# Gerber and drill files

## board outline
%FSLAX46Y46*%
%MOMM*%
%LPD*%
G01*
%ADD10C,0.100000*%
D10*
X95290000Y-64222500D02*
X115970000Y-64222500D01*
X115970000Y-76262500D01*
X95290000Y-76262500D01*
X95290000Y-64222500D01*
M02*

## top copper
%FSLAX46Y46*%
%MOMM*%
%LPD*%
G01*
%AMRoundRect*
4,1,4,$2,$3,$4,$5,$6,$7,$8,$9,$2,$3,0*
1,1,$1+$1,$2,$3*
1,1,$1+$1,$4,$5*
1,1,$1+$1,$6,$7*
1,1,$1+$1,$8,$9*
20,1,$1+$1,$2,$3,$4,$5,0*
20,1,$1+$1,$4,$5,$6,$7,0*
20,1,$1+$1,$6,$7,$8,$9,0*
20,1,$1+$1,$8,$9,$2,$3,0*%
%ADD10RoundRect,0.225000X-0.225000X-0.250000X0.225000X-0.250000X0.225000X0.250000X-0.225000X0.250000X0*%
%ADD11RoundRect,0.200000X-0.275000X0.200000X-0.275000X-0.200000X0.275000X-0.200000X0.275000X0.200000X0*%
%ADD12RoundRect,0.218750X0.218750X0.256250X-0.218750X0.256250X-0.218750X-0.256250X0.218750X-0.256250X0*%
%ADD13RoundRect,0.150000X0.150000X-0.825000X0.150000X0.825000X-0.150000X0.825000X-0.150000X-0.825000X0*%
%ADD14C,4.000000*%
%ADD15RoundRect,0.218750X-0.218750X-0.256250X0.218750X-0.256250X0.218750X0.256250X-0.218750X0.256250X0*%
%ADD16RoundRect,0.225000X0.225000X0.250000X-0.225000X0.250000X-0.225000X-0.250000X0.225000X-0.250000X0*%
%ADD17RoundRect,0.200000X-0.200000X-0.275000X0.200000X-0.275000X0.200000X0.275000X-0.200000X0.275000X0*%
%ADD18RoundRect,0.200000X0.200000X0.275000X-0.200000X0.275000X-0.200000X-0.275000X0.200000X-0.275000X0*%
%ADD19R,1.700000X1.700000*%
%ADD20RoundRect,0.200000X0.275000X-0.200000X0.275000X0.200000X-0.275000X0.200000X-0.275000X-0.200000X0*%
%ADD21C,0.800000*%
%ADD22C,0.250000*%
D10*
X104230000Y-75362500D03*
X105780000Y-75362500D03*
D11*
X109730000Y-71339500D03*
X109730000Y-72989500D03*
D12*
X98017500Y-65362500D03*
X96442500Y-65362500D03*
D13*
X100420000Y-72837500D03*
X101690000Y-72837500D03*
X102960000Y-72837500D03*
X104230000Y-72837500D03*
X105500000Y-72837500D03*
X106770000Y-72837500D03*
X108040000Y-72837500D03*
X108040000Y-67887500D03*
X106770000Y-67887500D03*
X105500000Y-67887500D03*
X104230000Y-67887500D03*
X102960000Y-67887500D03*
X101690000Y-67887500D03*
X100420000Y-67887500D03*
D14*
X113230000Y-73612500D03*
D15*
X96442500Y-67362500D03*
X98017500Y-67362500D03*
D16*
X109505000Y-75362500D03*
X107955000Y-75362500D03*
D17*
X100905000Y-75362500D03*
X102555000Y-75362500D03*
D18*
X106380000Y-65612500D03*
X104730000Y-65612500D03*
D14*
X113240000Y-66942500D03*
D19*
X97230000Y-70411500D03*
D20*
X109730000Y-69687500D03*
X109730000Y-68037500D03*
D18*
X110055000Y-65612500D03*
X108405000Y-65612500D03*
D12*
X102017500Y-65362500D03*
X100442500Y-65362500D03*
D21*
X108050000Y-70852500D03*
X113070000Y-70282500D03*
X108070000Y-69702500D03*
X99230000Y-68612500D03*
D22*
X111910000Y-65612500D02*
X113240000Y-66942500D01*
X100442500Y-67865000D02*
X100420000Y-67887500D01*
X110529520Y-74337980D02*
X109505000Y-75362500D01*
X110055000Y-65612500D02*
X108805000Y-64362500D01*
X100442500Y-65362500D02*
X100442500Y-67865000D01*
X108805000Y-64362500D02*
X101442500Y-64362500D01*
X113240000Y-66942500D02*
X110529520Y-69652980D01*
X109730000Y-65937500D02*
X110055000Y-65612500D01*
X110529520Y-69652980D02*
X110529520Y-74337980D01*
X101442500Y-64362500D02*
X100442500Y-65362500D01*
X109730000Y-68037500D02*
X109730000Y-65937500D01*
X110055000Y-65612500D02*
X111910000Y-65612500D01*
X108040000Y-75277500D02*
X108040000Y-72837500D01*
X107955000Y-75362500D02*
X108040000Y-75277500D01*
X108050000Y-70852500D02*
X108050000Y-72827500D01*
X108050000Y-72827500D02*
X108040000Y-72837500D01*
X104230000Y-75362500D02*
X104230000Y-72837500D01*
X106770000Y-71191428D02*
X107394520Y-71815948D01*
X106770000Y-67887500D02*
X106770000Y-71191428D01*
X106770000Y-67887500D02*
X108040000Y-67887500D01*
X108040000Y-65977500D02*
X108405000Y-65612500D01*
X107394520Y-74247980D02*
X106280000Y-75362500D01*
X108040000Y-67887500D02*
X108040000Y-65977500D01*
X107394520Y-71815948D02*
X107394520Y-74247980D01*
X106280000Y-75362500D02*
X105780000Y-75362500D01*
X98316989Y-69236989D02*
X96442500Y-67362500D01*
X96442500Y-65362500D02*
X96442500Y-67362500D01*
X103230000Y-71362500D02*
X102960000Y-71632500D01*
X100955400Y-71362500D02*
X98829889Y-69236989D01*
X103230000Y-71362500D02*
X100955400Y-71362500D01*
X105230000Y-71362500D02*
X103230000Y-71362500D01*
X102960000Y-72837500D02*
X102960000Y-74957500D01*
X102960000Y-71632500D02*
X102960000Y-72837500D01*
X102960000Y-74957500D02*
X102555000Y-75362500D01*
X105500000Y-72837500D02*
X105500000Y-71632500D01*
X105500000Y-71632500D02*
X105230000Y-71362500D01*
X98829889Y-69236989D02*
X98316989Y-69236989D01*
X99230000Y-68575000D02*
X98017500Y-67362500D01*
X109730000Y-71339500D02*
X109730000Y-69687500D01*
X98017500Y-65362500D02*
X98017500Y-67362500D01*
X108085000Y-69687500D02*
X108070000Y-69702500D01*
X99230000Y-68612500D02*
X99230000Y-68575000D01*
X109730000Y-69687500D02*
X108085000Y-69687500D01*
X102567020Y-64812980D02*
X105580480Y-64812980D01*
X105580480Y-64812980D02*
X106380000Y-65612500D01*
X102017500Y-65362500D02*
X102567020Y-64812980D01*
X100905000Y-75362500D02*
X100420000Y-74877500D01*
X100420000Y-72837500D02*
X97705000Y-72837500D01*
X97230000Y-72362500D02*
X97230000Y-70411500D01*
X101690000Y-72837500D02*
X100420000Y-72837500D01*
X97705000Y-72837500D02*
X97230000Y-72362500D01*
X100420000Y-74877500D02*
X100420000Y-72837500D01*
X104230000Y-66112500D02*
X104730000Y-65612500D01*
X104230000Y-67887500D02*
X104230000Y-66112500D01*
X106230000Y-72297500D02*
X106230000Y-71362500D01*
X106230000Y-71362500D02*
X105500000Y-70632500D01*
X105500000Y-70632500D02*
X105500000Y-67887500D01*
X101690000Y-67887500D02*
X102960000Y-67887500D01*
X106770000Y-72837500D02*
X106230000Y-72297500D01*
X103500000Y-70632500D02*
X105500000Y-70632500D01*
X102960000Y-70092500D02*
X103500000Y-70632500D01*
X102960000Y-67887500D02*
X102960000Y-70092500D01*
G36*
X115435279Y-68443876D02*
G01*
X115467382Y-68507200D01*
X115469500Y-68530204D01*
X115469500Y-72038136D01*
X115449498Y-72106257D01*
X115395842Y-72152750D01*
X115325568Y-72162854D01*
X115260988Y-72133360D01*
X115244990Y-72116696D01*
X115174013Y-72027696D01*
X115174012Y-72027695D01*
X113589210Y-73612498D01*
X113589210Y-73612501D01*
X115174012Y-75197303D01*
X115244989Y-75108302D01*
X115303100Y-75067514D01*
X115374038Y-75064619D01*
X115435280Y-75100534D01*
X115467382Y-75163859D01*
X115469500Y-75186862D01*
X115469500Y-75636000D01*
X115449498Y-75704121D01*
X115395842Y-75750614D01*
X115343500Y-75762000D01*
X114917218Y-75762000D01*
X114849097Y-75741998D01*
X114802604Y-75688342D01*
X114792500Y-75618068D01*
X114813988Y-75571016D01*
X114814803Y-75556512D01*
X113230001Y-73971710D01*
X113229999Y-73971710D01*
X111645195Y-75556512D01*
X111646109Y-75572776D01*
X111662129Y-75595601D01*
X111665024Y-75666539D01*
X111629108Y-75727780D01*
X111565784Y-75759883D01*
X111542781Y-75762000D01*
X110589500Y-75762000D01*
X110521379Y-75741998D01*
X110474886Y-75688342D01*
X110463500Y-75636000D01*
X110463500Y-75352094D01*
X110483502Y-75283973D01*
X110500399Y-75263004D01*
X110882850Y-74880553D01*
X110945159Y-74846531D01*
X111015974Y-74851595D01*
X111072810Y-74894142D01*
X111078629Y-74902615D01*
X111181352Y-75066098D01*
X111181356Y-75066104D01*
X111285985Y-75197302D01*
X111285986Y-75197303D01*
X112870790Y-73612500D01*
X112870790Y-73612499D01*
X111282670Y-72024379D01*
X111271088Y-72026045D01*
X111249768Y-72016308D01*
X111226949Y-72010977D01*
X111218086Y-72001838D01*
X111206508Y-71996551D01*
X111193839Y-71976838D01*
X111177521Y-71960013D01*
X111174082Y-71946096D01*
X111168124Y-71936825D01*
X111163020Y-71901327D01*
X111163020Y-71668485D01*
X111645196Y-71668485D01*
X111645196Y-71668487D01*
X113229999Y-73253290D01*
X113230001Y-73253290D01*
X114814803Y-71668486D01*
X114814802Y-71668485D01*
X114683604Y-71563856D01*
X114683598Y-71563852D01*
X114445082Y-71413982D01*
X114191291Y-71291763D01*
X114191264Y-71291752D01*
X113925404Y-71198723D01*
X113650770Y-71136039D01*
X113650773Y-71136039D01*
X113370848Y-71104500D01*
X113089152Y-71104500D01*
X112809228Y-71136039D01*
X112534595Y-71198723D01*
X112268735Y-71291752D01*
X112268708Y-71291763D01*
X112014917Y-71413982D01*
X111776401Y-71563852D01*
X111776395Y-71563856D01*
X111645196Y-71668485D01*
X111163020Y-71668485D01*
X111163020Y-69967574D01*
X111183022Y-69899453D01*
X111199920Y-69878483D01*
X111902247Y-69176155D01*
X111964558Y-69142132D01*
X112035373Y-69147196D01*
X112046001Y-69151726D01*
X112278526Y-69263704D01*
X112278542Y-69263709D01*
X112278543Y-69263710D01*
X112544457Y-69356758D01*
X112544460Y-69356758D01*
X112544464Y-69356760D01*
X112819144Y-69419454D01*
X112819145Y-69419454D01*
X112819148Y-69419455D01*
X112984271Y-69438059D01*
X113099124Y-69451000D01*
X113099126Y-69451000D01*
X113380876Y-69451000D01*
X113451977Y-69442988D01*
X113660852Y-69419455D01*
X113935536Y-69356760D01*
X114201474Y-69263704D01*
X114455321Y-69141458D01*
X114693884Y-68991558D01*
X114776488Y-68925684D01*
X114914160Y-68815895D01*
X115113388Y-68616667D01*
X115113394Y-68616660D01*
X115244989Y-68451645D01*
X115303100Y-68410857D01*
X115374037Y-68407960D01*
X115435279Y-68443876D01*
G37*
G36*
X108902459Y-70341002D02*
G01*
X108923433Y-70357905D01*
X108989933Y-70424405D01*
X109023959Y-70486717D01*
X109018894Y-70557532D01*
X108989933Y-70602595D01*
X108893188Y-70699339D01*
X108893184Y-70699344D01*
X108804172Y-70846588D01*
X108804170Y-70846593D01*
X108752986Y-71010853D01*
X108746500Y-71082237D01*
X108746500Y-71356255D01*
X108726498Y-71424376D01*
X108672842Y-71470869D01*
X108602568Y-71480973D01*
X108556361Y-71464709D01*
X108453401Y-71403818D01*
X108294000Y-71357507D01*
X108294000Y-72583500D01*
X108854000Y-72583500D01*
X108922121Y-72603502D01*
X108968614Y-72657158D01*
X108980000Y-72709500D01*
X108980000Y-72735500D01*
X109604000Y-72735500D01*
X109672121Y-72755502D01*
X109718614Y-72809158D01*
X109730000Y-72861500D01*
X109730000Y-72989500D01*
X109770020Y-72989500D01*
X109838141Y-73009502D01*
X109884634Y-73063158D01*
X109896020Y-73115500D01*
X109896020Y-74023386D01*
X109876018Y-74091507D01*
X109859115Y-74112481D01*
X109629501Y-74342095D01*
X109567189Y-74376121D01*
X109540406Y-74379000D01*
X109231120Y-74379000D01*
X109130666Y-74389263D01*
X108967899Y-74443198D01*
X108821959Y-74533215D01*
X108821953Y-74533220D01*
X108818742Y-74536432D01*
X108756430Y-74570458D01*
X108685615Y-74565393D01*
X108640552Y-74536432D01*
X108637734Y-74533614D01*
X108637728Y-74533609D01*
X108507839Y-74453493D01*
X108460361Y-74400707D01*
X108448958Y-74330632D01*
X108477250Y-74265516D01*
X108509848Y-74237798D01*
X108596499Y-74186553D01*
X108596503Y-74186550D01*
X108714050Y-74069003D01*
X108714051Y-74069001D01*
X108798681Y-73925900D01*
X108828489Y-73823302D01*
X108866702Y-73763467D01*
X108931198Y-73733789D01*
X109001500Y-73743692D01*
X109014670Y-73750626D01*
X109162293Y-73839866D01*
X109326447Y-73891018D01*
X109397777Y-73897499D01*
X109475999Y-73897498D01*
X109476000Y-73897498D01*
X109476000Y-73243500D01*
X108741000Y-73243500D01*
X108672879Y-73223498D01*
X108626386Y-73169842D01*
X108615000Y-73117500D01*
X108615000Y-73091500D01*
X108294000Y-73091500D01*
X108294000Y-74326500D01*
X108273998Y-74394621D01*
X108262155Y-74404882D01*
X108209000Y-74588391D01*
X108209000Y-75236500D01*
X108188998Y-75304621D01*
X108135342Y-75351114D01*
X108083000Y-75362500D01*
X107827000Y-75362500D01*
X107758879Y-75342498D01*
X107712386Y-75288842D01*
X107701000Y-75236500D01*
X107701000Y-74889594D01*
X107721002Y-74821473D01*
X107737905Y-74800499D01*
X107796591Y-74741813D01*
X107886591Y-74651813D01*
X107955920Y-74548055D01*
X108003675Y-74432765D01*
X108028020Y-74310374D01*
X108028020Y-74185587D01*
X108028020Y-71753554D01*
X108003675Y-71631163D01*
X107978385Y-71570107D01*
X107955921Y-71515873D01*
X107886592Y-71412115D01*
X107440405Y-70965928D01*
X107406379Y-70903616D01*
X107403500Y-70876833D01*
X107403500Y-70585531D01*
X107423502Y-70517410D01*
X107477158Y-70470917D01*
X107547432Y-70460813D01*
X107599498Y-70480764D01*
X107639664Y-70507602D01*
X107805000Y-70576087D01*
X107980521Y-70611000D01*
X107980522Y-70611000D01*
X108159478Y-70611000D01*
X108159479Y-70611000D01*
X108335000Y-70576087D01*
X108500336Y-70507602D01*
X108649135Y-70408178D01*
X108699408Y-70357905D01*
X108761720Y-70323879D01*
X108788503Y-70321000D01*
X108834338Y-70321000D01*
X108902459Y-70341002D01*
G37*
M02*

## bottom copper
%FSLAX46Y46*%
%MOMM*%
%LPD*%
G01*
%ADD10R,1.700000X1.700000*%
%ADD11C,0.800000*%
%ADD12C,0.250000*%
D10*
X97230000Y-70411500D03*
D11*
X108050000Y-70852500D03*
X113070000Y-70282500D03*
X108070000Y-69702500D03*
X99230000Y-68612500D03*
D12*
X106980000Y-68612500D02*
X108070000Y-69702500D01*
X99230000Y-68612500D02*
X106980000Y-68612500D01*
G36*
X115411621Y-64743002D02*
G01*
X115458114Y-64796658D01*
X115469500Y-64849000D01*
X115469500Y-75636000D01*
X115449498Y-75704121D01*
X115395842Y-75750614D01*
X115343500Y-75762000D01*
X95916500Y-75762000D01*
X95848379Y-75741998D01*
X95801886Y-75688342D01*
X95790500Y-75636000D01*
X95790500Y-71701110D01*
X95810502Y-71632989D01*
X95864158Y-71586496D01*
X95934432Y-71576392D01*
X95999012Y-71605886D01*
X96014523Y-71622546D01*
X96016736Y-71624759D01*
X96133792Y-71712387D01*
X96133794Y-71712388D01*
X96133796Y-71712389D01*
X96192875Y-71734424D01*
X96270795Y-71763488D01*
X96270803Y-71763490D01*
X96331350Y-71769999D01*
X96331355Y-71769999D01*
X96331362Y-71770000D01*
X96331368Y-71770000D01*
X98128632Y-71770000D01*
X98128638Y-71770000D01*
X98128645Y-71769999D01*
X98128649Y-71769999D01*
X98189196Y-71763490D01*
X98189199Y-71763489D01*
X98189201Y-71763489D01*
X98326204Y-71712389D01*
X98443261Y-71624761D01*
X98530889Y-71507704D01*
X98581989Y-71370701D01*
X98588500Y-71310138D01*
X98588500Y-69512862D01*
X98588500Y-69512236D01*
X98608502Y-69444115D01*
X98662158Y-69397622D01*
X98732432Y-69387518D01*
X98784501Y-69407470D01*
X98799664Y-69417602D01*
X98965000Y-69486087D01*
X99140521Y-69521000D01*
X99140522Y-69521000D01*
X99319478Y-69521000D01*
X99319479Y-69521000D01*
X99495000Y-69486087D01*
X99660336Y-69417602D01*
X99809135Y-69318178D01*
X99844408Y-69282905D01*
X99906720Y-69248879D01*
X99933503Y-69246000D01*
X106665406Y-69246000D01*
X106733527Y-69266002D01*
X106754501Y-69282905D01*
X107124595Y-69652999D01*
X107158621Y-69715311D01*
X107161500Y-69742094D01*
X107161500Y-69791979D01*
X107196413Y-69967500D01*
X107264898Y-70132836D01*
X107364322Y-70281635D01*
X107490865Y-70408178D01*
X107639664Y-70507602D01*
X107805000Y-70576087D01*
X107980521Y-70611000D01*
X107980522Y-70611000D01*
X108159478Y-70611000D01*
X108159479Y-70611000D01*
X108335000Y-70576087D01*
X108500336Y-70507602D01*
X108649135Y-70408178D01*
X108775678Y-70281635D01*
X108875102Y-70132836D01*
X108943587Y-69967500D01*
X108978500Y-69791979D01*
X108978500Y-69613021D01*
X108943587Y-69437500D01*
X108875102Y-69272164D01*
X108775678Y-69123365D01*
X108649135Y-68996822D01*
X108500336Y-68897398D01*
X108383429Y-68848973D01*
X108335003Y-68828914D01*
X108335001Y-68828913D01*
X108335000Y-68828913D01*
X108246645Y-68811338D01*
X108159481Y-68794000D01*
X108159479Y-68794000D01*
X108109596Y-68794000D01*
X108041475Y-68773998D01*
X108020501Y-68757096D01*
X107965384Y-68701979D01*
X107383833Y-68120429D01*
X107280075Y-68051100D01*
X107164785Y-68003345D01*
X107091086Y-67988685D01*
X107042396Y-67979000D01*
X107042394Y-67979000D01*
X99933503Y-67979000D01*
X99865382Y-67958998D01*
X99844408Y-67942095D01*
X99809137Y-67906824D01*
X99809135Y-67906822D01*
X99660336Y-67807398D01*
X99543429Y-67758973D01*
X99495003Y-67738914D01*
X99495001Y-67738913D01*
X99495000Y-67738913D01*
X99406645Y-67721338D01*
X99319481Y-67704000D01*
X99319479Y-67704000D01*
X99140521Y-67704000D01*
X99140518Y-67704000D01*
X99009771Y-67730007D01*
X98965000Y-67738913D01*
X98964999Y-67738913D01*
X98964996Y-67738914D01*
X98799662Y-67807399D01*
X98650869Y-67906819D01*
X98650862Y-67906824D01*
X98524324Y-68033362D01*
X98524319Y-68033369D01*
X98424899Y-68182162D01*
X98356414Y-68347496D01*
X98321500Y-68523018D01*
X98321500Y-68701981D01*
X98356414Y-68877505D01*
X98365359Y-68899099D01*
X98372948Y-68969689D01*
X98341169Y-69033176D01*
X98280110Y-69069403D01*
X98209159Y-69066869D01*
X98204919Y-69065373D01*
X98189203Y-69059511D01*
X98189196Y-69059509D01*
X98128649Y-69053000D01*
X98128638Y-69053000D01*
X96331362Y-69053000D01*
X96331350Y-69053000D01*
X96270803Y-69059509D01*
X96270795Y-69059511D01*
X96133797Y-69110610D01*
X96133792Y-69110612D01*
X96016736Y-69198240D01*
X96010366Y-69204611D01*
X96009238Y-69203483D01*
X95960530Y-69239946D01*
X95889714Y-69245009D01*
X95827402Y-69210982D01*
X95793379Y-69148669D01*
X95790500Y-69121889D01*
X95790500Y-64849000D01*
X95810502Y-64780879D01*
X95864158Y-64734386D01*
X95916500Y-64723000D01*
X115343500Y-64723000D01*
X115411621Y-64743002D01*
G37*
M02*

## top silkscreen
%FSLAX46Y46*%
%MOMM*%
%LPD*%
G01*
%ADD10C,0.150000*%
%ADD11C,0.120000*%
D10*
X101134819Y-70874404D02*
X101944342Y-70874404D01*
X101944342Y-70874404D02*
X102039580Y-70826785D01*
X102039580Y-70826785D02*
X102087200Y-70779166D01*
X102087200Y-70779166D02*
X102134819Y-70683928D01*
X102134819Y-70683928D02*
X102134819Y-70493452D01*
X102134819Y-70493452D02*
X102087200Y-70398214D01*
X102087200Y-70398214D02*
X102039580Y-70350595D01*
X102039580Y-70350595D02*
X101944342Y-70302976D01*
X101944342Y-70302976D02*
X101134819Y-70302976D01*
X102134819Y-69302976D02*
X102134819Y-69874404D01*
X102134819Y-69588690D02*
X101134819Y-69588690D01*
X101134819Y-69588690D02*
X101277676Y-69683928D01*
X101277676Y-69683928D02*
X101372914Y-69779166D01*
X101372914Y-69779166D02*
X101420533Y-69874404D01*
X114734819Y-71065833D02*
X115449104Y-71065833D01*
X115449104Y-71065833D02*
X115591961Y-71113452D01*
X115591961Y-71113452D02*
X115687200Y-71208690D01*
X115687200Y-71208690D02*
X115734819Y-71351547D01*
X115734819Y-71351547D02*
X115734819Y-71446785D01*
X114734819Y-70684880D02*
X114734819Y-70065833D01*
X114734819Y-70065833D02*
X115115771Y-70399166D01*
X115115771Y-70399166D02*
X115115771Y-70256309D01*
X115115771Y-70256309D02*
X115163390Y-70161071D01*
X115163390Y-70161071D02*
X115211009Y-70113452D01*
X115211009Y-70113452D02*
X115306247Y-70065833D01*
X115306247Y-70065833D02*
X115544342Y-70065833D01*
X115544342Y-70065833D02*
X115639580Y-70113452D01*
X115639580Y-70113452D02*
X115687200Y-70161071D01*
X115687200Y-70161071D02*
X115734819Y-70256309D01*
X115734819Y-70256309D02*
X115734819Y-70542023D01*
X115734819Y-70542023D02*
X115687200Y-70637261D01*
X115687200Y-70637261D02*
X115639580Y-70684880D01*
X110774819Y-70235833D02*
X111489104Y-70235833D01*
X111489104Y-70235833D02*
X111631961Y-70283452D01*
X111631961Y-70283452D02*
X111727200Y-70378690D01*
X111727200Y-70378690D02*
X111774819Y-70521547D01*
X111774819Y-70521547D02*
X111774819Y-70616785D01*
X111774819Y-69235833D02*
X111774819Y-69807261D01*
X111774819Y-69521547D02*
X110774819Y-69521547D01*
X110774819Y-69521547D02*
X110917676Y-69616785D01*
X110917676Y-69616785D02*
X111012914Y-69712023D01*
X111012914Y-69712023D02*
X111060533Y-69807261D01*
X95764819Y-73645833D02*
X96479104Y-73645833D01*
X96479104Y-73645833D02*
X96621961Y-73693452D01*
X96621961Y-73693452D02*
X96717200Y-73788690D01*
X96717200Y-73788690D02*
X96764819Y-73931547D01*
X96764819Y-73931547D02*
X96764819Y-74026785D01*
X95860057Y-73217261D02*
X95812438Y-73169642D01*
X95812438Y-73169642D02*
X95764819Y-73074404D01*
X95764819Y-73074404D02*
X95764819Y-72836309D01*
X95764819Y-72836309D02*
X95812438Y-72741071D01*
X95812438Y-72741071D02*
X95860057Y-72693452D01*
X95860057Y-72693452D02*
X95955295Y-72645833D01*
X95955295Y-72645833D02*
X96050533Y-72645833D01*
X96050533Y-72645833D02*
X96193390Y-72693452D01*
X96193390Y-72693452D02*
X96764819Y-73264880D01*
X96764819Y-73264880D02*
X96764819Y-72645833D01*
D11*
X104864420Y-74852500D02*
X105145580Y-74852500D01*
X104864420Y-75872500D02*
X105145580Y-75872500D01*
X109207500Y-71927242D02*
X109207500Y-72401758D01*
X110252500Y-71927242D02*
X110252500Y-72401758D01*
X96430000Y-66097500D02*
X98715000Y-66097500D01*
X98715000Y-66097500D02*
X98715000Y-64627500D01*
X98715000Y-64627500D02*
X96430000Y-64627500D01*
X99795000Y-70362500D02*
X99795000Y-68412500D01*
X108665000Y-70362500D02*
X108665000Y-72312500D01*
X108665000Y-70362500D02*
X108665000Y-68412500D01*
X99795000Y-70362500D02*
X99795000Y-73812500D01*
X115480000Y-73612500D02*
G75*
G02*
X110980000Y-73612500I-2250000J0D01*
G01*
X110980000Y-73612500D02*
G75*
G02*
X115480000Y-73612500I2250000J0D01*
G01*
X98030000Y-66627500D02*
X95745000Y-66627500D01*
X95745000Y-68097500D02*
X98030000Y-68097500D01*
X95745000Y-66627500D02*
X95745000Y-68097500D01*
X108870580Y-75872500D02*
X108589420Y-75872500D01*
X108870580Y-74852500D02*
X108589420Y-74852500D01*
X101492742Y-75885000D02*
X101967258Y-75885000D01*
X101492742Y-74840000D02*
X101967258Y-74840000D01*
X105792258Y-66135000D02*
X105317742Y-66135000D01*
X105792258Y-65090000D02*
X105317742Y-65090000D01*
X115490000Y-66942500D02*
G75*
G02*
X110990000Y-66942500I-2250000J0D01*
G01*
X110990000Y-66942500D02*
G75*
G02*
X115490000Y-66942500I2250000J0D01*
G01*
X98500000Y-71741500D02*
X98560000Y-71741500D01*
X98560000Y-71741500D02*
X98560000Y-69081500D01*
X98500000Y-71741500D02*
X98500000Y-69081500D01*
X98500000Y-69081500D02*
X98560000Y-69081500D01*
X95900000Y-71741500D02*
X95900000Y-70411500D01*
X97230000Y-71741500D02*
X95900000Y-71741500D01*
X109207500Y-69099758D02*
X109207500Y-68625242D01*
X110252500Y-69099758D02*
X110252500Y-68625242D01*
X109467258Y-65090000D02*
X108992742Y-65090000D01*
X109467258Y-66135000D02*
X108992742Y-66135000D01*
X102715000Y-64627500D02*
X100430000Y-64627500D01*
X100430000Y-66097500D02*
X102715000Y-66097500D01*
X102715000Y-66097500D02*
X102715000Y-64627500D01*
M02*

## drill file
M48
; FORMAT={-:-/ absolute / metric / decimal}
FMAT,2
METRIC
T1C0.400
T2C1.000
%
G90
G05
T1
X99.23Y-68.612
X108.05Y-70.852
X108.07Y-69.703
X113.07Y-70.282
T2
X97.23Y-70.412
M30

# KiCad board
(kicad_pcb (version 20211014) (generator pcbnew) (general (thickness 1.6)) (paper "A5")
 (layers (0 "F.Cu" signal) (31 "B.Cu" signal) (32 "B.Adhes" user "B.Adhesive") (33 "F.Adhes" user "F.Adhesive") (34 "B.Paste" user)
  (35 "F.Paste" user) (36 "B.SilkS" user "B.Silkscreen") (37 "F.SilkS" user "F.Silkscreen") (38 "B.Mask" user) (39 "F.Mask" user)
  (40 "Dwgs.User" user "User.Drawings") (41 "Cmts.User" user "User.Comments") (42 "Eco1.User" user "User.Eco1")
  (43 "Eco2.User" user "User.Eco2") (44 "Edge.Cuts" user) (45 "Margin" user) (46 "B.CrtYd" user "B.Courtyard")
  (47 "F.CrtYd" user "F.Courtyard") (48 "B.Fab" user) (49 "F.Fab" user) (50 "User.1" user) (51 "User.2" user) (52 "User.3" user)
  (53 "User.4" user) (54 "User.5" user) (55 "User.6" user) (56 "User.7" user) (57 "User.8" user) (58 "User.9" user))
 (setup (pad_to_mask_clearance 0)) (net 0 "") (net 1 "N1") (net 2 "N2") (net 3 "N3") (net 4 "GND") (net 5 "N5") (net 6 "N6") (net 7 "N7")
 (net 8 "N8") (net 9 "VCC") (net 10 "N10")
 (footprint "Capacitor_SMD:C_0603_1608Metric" (layer "F.Cu") (at 105.005 75.3625)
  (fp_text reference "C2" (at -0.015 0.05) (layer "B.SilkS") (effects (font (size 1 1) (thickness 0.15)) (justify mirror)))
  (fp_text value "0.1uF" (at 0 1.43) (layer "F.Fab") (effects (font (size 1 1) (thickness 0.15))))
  (fp_line (start -0.14058 -0.51) (end 0.14058 -0.51) (layer "F.SilkS") (width 0.12))
  (fp_line (start -0.14058 0.51) (end 0.14058 0.51) (layer "F.SilkS") (width 0.12))
  (pad "1" smd roundrect locked (at -0.775 0) (size 0.9 0.95) (layers "F.Cu" "F.Paste" "F.Mask") (roundrect_rratio 0.25) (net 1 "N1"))
  (pad "2" smd roundrect locked (at 0.775 0) (size 0.9 0.95) (layers "F.Cu" "F.Paste" "F.Mask") (roundrect_rratio 0.25) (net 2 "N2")))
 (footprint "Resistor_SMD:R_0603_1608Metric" (layer "F.Cu") (at 109.73 72.1645 -90)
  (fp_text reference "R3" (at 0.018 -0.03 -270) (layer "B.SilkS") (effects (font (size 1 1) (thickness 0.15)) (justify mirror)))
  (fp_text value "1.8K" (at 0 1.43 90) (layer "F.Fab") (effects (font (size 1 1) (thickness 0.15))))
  (fp_line (start -0.237258 0.5225) (end 0.237258 0.5225) (layer "F.SilkS") (width 0.12))
  (fp_line (start -0.237258 -0.5225) (end 0.237258 -0.5225) (layer "F.SilkS") (width 0.12))
  (pad "1" smd roundrect locked (at -0.825 0 270) (size 0.8 0.95) (layers "F.Cu" "F.Paste" "F.Mask") (roundrect_rratio 0.25) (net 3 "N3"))
  (pad "2" smd roundrect locked (at 0.825 0 270) (size 0.8 0.95) (layers "F.Cu" "F.Paste" "F.Mask") (roundrect_rratio 0.25) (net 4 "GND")))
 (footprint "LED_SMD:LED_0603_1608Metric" (layer "F.Cu") (at 97.23 65.3625 180)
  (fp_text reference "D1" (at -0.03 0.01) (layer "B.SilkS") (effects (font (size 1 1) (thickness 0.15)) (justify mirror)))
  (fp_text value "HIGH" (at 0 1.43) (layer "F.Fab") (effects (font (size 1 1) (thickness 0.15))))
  (fp_line (start 0.8 -0.735) (end -1.485 -0.735) (layer "F.SilkS") (width 0.12))
  (fp_line (start -1.485 -0.735) (end -1.485 0.735) (layer "F.SilkS") (width 0.12))
  (fp_line (start -1.485 0.735) (end 0.8 0.735) (layer "F.SilkS") (width 0.12))
  (pad "1" smd roundrect locked (at -0.7875 0 180) (size 0.875 0.95) (layers "F.Cu" "F.Paste" "F.Mask") (roundrect_rratio 0.25) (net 3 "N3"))
  (pad "2" smd roundrect locked (at 0.7875 0 180) (size 0.875 0.95) (layers "F.Cu" "F.Paste" "F.Mask") (roundrect_rratio 0.25) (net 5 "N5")))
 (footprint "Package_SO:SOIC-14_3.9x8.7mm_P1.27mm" (layer "F.Cu") (at 104.23 70.3625 90)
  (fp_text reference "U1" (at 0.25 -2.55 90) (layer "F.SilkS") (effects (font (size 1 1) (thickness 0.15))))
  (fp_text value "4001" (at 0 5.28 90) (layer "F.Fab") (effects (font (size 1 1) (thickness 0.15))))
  (fp_line (start 0 -4.435) (end 1.95 -4.435) (layer "F.SilkS") (width 0.12))
  (fp_line (start 0 4.435) (end -1.95 4.435) (layer "F.SilkS") (width 0.12))
  (fp_line (start 0 4.435) (end 1.95 4.435) (layer "F.SilkS") (width 0.12))
  (fp_line (start 0 -4.435) (end -3.45 -4.435) (layer "F.SilkS") (width 0.12))
  (pad "1" smd roundrect locked (at -2.475 -3.81 90) (size 1.95 0.6) (layers "F.Cu" "F.Paste" "F.Mask") (roundrect_rratio 0.25) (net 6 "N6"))
  (pad "2" smd roundrect locked (at -2.475 -2.54 90) (size 1.95 0.6) (layers "F.Cu" "F.Paste" "F.Mask") (roundrect_rratio 0.25) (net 6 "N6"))
  (pad "3" smd roundrect locked (at -2.475 -1.27 90) (size 1.95 0.6) (layers "F.Cu" "F.Paste" "F.Mask") (roundrect_rratio 0.25) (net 5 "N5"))
  (pad "4" smd roundrect locked (at -2.475 0 90) (size 1.95 0.6) (layers "F.Cu" "F.Paste" "F.Mask") (roundrect_rratio 0.25) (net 1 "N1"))
  (pad "5" smd roundrect locked (at -2.475 1.27 90) (size 1.95 0.6) (layers "F.Cu" "F.Paste" "F.Mask") (roundrect_rratio 0.25) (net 5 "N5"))
  (pad "6" smd roundrect locked (at -2.475 2.54 90) (size 1.95 0.6) (layers "F.Cu" "F.Paste" "F.Mask") (roundrect_rratio 0.25) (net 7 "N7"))
  (pad "7" smd roundrect locked (at -2.475 3.81 90) (size 1.95 0.6) (layers "F.Cu" "F.Paste" "F.Mask") (roundrect_rratio 0.25) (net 4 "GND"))
  (pad "8" smd roundrect locked (at 2.475 3.81 90) (size 1.95 0.6) (layers "F.Cu" "F.Paste" "F.Mask") (roundrect_rratio 0.25) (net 2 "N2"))
  (pad "9" smd roundrect locked (at 2.475 2.54 90) (size 1.95 0.6) (layers "F.Cu" "F.Paste" "F.Mask") (roundrect_rratio 0.25) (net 2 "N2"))
  (pad "10" smd roundrect locked (at 2.475 1.27 90) (size 1.95 0.6) (layers "F.Cu" "F.Paste" "F.Mask") (roundrect_rratio 0.25) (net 7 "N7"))
  (pad "11" smd roundrect locked (at 2.475 0 90) (size 1.95 0.6) (layers "F.Cu" "F.Paste" "F.Mask") (roundrect_rratio 0.25) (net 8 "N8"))
  (pad "12" smd roundrect locked (at 2.475 -1.27 90) (size 1.95 0.6) (layers "F.Cu" "F.Paste" "F.Mask") (roundrect_rratio 0.25) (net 7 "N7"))
  (pad "13" smd roundrect locked (at 2.475 -2.54 90) (size 1.95 0.6) (layers "F.Cu" "F.Paste" "F.Mask") (roundrect_rratio 0.25) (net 7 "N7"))
  (pad "14" smd roundrect locked (at 2.475 -3.81 90) (size 1.95 0.6) (layers "F.Cu" "F.Paste" "F.Mask") (roundrect_rratio 0.25)
   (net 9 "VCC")))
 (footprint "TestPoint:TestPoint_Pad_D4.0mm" (layer "F.Cu") (at 113.23 73.6125 90)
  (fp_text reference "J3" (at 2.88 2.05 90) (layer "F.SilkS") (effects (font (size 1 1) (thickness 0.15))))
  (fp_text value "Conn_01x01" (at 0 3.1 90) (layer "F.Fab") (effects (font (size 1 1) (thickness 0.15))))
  (fp_circle (center 0 0) (end 0 2.25) (layer "F.SilkS") (width 0.12) (fill none))
  (pad "1" smd circle locked (at 0 0 90) (size 4 4) (layers "F.Cu" "F.Mask") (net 4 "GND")))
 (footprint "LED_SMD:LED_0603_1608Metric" (layer "F.Cu") (at 97.23 67.3625)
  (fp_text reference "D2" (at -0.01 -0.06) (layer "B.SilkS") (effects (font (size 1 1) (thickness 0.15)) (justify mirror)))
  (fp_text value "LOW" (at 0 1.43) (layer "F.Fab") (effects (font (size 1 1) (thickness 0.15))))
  (fp_line (start 0.8 -0.735) (end -1.485 -0.735) (layer "F.SilkS") (width 0.12))
  (fp_line (start -1.485 0.735) (end 0.8 0.735) (layer "F.SilkS") (width 0.12))
  (fp_line (start -1.485 -0.735) (end -1.485 0.735) (layer "F.SilkS") (width 0.12))
  (pad "1" smd roundrect locked (at -0.7875 0) (size 0.875 0.95) (layers "F.Cu" "F.Paste" "F.Mask") (roundrect_rratio 0.25) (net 5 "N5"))
  (pad "2" smd roundrect locked (at 0.7875 0) (size 0.875 0.95) (layers "F.Cu" "F.Paste" "F.Mask") (roundrect_rratio 0.25) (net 3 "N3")))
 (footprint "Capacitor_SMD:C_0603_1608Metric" (layer "F.Cu") (at 108.73 75.3625 180)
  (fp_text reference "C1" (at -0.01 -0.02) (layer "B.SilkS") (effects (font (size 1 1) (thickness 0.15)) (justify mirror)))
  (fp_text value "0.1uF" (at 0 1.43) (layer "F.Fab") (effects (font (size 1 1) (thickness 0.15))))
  (fp_line (start -0.14058 -0.51) (end 0.14058 -0.51) (layer "F.SilkS") (width 0.12))
  (fp_line (start -0.14058 0.51) (end 0.14058 0.51) (layer "F.SilkS") (width 0.12))
  (pad "1" smd roundrect locked (at -0.775 0 180) (size 0.9 0.95) (layers "F.Cu" "F.Paste" "F.Mask") (roundrect_rratio 0.25) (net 9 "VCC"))
  (pad "2" smd roundrect locked (at 0.775 0 180) (size 0.9 0.95) (layers "F.Cu" "F.Paste" "F.Mask") (roundrect_rratio 0.25) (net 4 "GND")))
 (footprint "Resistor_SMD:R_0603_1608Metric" (layer "F.Cu") (at 101.73 75.3625)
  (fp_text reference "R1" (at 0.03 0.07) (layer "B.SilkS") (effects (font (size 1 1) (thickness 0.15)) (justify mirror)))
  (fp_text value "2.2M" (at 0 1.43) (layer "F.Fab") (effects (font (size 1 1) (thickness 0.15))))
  (fp_line (start -0.237258 0.5225) (end 0.237258 0.5225) (layer "F.SilkS") (width 0.12))
  (fp_line (start -0.237258 -0.5225) (end 0.237258 -0.5225) (layer "F.SilkS") (width 0.12))
  (pad "1" smd roundrect locked (at -0.825 0) (size 0.8 0.95) (layers "F.Cu" "F.Paste" "F.Mask") (roundrect_rratio 0.25) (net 6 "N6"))
  (pad "2" smd roundrect locked (at 0.825 0) (size 0.8 0.95) (layers "F.Cu" "F.Paste" "F.Mask") (roundrect_rratio 0.25) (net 5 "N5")))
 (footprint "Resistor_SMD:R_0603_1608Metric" (layer "F.Cu") (at 105.555 65.6125 180)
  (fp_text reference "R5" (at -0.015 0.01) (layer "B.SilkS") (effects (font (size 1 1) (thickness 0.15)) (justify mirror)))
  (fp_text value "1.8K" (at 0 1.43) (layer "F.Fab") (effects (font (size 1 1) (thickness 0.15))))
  (fp_line (start -0.237258 -0.5225) (end 0.237258 -0.5225) (layer "F.SilkS") (width 0.12))
  (fp_line (start -0.237258 0.5225) (end 0.237258 0.5225) (layer "F.SilkS") (width 0.12))
  (pad "1" smd roundrect locked (at -0.825 0 180) (size 0.8 0.95) (layers "F.Cu" "F.Paste" "F.Mask") (roundrect_rratio 0.25) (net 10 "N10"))
  (pad "2" smd roundrect locked (at 0.825 0 180) (size 0.8 0.95) (layers "F.Cu" "F.Paste" "F.Mask") (roundrect_rratio 0.25) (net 8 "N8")))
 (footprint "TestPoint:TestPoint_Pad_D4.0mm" (layer "F.Cu") (at 113.24 66.9425 90)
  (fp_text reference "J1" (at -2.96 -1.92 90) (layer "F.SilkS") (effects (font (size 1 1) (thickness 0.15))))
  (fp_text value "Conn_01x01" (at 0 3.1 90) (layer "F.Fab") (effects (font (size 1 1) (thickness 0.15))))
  (fp_circle (center 0 0) (end 0 2.25) (layer "F.SilkS") (width 0.12) (fill none))
  (pad "1" smd circle locked (at 0 0 90) (size 4 4) (layers "F.Cu" "F.Mask") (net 9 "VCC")))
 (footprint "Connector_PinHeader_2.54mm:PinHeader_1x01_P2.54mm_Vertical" (layer "F.Cu") (at 97.23 70.4115 90)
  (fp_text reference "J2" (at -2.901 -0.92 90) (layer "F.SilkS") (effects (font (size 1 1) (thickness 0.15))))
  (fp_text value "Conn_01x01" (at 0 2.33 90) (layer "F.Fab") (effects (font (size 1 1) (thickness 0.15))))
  (fp_line (start -1.33 1.27) (end -1.33 1.33) (layer "F.SilkS") (width 0.12))
  (fp_line (start -1.33 1.33) (end 1.33 1.33) (layer "F.SilkS") (width 0.12))
  (fp_line (start -1.33 1.27) (end 1.33 1.27) (layer "F.SilkS") (width 0.12))
  (fp_line (start 1.33 1.27) (end 1.33 1.33) (layer "F.SilkS") (width 0.12))
  (fp_line (start -1.33 -1.33) (end 0 -1.33) (layer "F.SilkS") (width 0.12))
  (fp_line (start -1.33 0) (end -1.33 -1.33) (layer "F.SilkS") (width 0.12))
  (pad "1" thru_hole rect locked (at 0 0 90) (size 1.7 1.7) (drill 1) (layers *.Cu *.Mask) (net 6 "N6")))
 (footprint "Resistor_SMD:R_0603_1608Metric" (layer "F.Cu") (at 109.73 68.8625 90)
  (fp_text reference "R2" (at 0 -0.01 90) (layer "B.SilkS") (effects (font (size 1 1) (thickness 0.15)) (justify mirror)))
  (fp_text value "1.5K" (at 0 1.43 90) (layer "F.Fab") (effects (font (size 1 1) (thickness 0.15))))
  (fp_line (start -0.237258 -0.5225) (end 0.237258 -0.5225) (layer "F.SilkS") (width 0.12))
  (fp_line (start -0.237258 0.5225) (end 0.237258 0.5225) (layer "F.SilkS") (width 0.12))
  (pad "1" smd roundrect locked (at -0.825 0 90) (size 0.8 0.95) (layers "F.Cu" "F.Paste" "F.Mask") (roundrect_rratio 0.25) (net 3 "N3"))
  (pad "2" smd roundrect locked (at 0.825 0 90) (size 0.8 0.95) (layers "F.Cu" "F.Paste" "F.Mask") (roundrect_rratio 0.25) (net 9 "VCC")))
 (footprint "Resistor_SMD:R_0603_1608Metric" (layer "F.Cu") (at 109.23 65.6125 180)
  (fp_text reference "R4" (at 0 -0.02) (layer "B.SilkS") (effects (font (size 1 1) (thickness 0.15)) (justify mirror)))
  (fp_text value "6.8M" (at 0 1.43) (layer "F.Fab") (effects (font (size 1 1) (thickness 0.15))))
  (fp_line (start -0.237258 0.5225) (end 0.237258 0.5225) (layer "F.SilkS") (width 0.12))
  (fp_line (start -0.237258 -0.5225) (end 0.237258 -0.5225) (layer "F.SilkS") (width 0.12))
  (pad "1" smd roundrect locked (at -0.825 0 180) (size 0.8 0.95) (layers "F.Cu" "F.Paste" "F.Mask") (roundrect_rratio 0.25) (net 9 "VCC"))
  (pad "2" smd roundrect locked (at 0.825 0 180) (size 0.8 0.95) (layers "F.Cu" "F.Paste" "F.Mask") (roundrect_rratio 0.25) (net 2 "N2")))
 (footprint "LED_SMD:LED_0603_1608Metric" (layer "F.Cu") (at 101.23 65.3625 180)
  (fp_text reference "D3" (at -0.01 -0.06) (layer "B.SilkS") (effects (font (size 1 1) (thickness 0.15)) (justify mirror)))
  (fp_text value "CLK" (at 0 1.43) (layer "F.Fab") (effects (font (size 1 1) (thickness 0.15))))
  (fp_line (start -1.485 0.735) (end 0.8 0.735) (layer "F.SilkS") (width 0.12))
  (fp_line (start 0.8 -0.735) (end -1.485 -0.735) (layer "F.SilkS") (width 0.12))
  (fp_line (start -1.485 -0.735) (end -1.485 0.735) (layer "F.SilkS") (width 0.12))
  (pad "1" smd roundrect locked (at -0.7875 0 180) (size 0.875 0.95) (layers "F.Cu" "F.Paste" "F.Mask") (roundrect_rratio 0.25)
   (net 10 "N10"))
  (pad "2" smd roundrect locked (at 0.7875 0 180) (size 0.875 0.95) (layers "F.Cu" "F.Paste" "F.Mask") (roundrect_rratio 0.25) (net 9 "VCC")))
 (gr_rect (start 95.29 64.2225) (end 115.97 76.2625) (layer "Edge.Cuts") (width 0.1) (fill none))
 (segment (start 111.91 65.6125) (end 113.24 66.9425) (width 0.25) (layer "F.Cu") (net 9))
 (segment (start 100.4425 67.865) (end 100.42 67.8875) (width 0.25) (layer "F.Cu") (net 9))
 (segment (start 110.52952 74.33798) (end 109.505 75.3625) (width 0.25) (layer "F.Cu") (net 9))
 (segment (start 110.055 65.6125) (end 108.805 64.3625) (width 0.25) (layer "F.Cu") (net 9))
 (segment (start 100.4425 65.3625) (end 100.4425 67.865) (width 0.25) (layer "F.Cu") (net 9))
 (segment (start 108.805 64.3625) (end 101.4425 64.3625) (width 0.25) (layer "F.Cu") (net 9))
 (segment (start 113.24 66.9425) (end 110.52952 69.65298) (width 0.25) (layer "F.Cu") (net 9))
 (segment (start 109.73 65.9375) (end 110.055 65.6125) (width 0.25) (layer "F.Cu") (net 9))
 (segment (start 110.52952 69.65298) (end 110.52952 74.33798) (width 0.25) (layer "F.Cu") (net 9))
 (segment (start 101.4425 64.3625) (end 100.4425 65.3625) (width 0.25) (layer "F.Cu") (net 9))
 (segment (start 109.73 68.0375) (end 109.73 65.9375) (width 0.25) (layer "F.Cu") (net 9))
 (segment (start 110.055 65.6125) (end 111.91 65.6125) (width 0.25) (layer "F.Cu") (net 9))
 (segment (start 108.04 75.2775) (end 108.04 72.8375) (width 0.25) (layer "F.Cu") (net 4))
 (segment (start 107.955 75.3625) (end 108.04 75.2775) (width 0.25) (layer "F.Cu") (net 4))
 (segment (start 108.05 70.8525) (end 108.05 72.8275) (width 0.25) (layer "F.Cu") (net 4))
 (segment (start 108.05 72.8275) (end 108.04 72.8375) (width 0.25) (layer "F.Cu") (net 4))
 (via (at 108.05 70.8525) (size 0.8) (drill 0.4) (layers "F.Cu" "B.Cu") (free) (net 4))
 (via (at 113.07 70.2825) (size 0.8) (drill 0.4) (layers "F.Cu" "B.Cu") (free) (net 4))
 (segment (start 104.23 75.3625) (end 104.23 72.8375) (width 0.25) (layer "F.Cu") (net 1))
 (segment (start 106.77 71.191428) (end 107.39452 71.815948) (width 0.25) (layer "F.Cu") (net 2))
 (segment (start 106.77 67.8875) (end 106.77 71.191428) (width 0.25) (layer "F.Cu") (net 2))
 (segment (start 106.77 67.8875) (end 108.04 67.8875) (width 0.25) (layer "F.Cu") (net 2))
 (segment (start 108.04 65.9775) (end 108.405 65.6125) (width 0.25) (layer "F.Cu") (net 2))
 (segment (start 107.39452 74.24798) (end 106.28 75.3625) (width 0.25) (layer "F.Cu") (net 2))
 (segment (start 108.04 67.8875) (end 108.04 65.9775) (width 0.25) (layer "F.Cu") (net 2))
 (segment (start 107.39452 71.815948) (end 107.39452 74.24798) (width 0.25) (layer "F.Cu") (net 2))
 (segment (start 106.28 75.3625) (end 105.78 75.3625) (width 0.25) (layer "F.Cu") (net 2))
 (segment (start 98.316989 69.236989) (end 96.4425 67.3625) (width 0.25) (layer "F.Cu") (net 5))
 (segment (start 96.4425 65.3625) (end 96.4425 67.3625) (width 0.25) (layer "F.Cu") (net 5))
 (segment (start 103.23 71.3625) (end 102.96 71.6325) (width 0.25) (layer "F.Cu") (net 5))
 (segment (start 100.9554 71.3625) (end 98.829889 69.236989) (width 0.25) (layer "F.Cu") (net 5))
 (segment (start 103.23 71.3625) (end 100.9554 71.3625) (width 0.25) (layer "F.Cu") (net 5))
 (segment (start 105.23 71.3625) (end 103.23 71.3625) (width 0.25) (layer "F.Cu") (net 5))
 (segment (start 102.96 72.8375) (end 102.96 74.9575) (width 0.25) (layer "F.Cu") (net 5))
 (segment (start 102.96 71.6325) (end 102.96 72.8375) (width 0.25) (layer "F.Cu") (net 5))
 (segment (start 102.96 74.9575) (end 102.555 75.3625) (width 0.25) (layer "F.Cu") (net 5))
 (segment (start 105.5 72.8375) (end 105.5 71.6325) (width 0.25) (layer "F.Cu") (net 5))
 (segment (start 105.5 71.6325) (end 105.23 71.3625) (width 0.25) (layer "F.Cu") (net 5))
 (segment (start 98.829889 69.236989) (end 98.316989 69.236989) (width 0.25) (layer "F.Cu") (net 5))
 (segment (start 99.23 68.575) (end 98.0175 67.3625) (width 0.25) (layer "F.Cu") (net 3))
 (segment (start 109.73 71.3395) (end 109.73 69.6875) (width 0.25) (layer "F.Cu") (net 3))
 (segment (start 98.0175 65.3625) (end 98.0175 67.3625) (width 0.25) (layer "F.Cu") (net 3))
 (segment (start 108.085 69.6875) (end 108.07 69.7025) (width 0.25) (layer "F.Cu") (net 3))
 (segment (start 99.23 68.6125) (end 99.23 68.575) (width 0.25) (layer "F.Cu") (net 3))
 (segment (start 109.73 69.6875) (end 108.085 69.6875) (width 0.25) (layer "F.Cu") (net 3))
 (via (at 108.07 69.7025) (size 0.8) (drill 0.4) (layers "F.Cu" "B.Cu") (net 3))
 (via (at 99.23 68.6125) (size 0.8) (drill 0.4) (layers "F.Cu" "B.Cu") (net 3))
 (segment (start 106.98 68.6125) (end 108.07 69.7025) (width 0.25) (layer "B.Cu") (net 3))
 (segment (start 99.23 68.6125) (end 106.98 68.6125) (width 0.25) (layer "B.Cu") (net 3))
 (segment (start 102.56702 64.81298) (end 105.58048 64.81298) (width 0.25) (layer "F.Cu") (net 10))
 (segment (start 105.58048 64.81298) (end 106.38 65.6125) (width 0.25) (layer "F.Cu") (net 10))
 (segment (start 102.0175 65.3625) (end 102.56702 64.81298) (width 0.25) (layer "F.Cu") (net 10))
 (segment (start 100.905 75.3625) (end 100.42 74.8775) (width 0.25) (layer "F.Cu") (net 6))
 (segment (start 100.42 72.8375) (end 97.705 72.8375) (width 0.25) (layer "F.Cu") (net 6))
 (segment (start 97.23 72.3625) (end 97.23 70.4115) (width 0.25) (layer "F.Cu") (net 6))
 (segment (start 101.69 72.8375) (end 100.42 72.8375) (width 0.25) (layer "F.Cu") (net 6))
 (segment (start 97.705 72.8375) (end 97.23 72.3625) (width 0.25) (layer "F.Cu") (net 6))
 (segment (start 100.42 74.8775) (end 100.42 72.8375) (width 0.25) (layer "F.Cu") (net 6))
 (segment (start 104.23 66.1125) (end 104.73 65.6125) (width 0.25) (layer "F.Cu") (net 8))
 (segment (start 104.23 67.8875) (end 104.23 66.1125) (width 0.25) (layer "F.Cu") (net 8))
 (segment (start 106.23 72.2975) (end 106.23 71.3625) (width 0.25) (layer "F.Cu") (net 7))
 (segment (start 106.23 71.3625) (end 105.5 70.6325) (width 0.25) (layer "F.Cu") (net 7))
 (segment (start 105.5 70.6325) (end 105.5 67.8875) (width 0.25) (layer "F.Cu") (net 7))
 (segment (start 101.69 67.8875) (end 102.96 67.8875) (width 0.25) (layer "F.Cu") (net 7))
 (segment (start 106.77 72.8375) (end 106.23 72.2975) (width 0.25) (layer "F.Cu") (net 7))
 (segment (start 103.5 70.6325) (end 105.5 70.6325) (width 0.25) (layer "F.Cu") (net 7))
 (segment (start 102.96 70.0925) (end 103.5 70.6325) (width 0.25) (layer "F.Cu") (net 7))
 (segment (start 102.96 67.8875) (end 102.96 70.0925) (width 0.25) (layer "F.Cu") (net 7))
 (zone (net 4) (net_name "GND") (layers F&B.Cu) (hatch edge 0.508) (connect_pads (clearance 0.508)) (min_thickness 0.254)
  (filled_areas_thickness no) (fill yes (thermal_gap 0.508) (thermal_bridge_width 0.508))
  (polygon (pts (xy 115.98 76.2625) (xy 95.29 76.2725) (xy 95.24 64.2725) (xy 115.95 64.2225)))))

